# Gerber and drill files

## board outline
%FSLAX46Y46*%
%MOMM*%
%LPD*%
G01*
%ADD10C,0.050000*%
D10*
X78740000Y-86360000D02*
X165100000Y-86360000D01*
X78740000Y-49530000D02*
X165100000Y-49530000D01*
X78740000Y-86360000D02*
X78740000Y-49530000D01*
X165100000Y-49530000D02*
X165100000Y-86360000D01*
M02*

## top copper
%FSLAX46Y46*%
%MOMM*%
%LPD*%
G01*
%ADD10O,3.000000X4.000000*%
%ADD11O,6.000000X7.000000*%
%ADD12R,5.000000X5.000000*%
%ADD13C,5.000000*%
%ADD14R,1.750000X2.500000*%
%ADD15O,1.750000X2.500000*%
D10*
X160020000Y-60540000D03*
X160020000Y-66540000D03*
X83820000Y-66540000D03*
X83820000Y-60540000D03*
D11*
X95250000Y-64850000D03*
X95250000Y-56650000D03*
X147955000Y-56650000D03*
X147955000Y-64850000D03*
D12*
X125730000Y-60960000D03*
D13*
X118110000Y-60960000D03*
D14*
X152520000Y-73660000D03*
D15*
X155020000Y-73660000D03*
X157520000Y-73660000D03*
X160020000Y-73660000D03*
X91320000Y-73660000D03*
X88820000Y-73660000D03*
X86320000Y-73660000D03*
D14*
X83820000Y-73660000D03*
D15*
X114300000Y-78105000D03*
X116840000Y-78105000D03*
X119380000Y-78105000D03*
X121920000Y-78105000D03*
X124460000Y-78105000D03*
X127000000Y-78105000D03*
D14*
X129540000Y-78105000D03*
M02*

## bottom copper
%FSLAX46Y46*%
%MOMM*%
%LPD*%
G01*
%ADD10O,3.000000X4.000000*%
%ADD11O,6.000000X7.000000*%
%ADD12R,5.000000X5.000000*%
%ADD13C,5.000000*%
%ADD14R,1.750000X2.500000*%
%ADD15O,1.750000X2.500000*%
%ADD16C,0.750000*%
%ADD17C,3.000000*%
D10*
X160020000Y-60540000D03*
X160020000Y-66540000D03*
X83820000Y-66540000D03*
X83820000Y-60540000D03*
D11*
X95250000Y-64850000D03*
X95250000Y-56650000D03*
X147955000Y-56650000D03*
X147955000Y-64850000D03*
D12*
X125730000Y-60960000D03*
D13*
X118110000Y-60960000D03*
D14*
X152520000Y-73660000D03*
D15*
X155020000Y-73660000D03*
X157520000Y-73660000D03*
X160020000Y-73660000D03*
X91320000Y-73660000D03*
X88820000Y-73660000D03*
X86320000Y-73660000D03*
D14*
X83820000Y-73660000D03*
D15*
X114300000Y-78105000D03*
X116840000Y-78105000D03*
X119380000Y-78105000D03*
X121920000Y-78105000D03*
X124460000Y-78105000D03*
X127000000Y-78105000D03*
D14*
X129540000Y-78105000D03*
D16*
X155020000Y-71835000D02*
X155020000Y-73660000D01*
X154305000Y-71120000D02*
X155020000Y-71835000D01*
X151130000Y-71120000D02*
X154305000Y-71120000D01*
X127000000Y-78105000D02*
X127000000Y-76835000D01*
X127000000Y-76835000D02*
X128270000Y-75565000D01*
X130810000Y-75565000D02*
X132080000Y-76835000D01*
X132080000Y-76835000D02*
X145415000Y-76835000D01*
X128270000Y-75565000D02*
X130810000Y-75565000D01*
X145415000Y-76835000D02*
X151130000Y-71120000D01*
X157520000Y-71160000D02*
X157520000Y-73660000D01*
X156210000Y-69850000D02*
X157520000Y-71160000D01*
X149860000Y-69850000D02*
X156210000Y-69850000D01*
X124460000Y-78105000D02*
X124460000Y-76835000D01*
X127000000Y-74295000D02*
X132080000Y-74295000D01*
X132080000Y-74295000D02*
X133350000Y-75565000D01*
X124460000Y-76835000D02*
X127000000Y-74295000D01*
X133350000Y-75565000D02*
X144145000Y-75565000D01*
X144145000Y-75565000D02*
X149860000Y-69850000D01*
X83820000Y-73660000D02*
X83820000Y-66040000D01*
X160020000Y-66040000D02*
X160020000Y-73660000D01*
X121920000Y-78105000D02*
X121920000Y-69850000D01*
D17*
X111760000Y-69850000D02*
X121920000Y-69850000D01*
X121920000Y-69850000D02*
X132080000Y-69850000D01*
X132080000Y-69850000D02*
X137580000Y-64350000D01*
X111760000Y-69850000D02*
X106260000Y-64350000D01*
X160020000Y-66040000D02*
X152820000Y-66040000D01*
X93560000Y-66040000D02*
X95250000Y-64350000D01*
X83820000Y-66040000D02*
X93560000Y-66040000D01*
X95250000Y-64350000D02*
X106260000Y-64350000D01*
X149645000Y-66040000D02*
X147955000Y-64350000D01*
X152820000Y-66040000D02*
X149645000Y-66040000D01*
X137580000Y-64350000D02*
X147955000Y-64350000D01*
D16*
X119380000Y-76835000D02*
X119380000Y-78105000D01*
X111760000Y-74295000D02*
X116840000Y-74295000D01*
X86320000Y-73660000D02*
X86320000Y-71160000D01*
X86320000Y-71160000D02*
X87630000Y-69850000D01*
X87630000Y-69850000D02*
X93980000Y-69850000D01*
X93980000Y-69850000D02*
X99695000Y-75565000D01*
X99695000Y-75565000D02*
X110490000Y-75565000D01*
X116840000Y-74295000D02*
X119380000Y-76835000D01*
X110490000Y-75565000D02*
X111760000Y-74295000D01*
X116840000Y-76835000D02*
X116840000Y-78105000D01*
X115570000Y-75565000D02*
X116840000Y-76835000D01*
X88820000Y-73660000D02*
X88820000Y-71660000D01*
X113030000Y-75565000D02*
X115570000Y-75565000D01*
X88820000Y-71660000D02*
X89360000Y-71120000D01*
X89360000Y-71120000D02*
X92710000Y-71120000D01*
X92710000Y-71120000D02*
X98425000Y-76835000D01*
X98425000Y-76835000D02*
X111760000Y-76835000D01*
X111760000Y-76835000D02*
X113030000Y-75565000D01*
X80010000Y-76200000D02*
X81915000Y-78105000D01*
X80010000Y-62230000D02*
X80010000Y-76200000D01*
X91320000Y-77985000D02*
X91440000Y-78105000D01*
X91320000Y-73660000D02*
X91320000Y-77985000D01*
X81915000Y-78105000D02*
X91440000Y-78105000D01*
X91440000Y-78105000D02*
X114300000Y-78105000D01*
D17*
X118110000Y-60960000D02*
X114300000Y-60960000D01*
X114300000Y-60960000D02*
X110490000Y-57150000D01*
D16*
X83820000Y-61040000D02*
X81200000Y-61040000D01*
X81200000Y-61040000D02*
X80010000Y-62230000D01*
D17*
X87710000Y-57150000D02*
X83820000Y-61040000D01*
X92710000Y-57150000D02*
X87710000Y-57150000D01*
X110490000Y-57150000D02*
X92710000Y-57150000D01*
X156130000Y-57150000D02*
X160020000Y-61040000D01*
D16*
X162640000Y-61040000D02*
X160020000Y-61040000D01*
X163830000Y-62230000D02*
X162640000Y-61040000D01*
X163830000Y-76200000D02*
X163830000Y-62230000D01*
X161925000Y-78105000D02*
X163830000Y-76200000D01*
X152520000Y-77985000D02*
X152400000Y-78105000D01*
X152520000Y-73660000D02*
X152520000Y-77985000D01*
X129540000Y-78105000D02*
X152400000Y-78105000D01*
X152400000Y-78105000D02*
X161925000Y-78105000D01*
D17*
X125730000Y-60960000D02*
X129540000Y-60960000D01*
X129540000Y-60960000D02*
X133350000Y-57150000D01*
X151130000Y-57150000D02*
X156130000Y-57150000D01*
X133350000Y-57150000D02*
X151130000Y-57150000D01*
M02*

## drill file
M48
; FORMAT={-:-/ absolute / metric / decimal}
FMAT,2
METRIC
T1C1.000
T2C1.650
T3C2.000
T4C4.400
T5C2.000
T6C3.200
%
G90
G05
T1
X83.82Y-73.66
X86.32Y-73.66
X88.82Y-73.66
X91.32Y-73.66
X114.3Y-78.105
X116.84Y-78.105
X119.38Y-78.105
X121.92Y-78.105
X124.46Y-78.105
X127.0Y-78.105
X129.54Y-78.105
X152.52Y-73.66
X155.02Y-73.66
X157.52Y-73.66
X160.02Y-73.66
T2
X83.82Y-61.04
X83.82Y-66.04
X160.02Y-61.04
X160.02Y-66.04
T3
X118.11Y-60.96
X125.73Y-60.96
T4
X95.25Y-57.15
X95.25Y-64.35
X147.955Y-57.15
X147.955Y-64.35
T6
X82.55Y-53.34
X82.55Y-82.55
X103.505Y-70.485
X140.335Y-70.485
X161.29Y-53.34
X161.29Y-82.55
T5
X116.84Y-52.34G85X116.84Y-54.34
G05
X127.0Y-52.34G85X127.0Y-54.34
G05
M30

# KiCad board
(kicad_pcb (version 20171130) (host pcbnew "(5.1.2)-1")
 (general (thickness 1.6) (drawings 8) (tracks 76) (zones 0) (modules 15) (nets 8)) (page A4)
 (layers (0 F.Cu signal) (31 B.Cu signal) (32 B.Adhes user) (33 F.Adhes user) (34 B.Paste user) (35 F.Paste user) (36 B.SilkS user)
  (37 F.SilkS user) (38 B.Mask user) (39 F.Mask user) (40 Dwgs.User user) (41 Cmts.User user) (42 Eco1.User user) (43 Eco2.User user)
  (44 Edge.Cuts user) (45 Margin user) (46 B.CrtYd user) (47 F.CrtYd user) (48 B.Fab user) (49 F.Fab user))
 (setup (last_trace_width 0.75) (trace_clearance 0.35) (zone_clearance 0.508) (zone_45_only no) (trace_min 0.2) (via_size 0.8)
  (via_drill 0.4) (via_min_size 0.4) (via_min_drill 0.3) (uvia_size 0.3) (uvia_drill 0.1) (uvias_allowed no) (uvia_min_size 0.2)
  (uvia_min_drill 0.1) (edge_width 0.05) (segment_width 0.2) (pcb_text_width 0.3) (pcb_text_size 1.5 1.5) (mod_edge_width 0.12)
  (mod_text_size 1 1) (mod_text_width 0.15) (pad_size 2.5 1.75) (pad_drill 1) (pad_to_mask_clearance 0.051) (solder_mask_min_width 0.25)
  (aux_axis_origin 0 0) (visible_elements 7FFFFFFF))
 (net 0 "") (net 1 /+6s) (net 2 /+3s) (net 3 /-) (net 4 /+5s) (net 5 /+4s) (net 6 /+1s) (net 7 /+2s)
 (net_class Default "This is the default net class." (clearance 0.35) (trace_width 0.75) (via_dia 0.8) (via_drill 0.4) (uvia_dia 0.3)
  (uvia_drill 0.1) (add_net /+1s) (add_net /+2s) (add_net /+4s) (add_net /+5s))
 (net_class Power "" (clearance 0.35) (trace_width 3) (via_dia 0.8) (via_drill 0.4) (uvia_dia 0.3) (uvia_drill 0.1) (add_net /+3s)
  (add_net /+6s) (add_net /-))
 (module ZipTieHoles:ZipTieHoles (layer F.Cu) (at 121.92 53.34)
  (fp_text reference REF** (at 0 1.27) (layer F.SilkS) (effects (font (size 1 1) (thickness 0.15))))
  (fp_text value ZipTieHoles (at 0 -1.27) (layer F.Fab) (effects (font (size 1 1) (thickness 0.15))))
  (pad "" np_thru_hole oval (at 5.08 0) (size 2 4) (drill oval 2 4) (layers *.Cu *.Mask))
  (pad "" np_thru_hole oval (at -5.08 0) (size 2 4) (drill oval 2 4) (layers *.Cu *.Mask)))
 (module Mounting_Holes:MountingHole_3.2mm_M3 (layer F.Cu) (at 140.335 70.485)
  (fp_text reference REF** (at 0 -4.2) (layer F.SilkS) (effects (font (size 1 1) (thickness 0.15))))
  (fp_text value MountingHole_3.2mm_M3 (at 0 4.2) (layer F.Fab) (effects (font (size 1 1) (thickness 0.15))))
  (pad 1 np_thru_hole circle (at 0 0) (size 3.2 3.2) (drill 3.2) (layers *.Cu *.Mask)))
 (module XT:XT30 (layer F.Cu) (at 160.02 63.54 90)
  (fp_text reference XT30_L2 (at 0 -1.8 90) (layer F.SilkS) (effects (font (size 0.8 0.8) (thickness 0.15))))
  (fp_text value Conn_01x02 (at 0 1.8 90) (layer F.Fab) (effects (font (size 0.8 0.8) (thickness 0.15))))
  (pad 1 thru_hole oval (at 2.5 0 90) (size 4 3) (drill 1.65 (offset 0.5 0)) (layers *.Cu *.Mask) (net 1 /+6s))
  (pad 2 thru_hole oval (at -2.5 0 90) (size 4 3) (drill 1.65 (offset -0.5 0)) (layers *.Cu *.Mask) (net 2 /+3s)))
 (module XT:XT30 (layer F.Cu) (at 83.82 63.54 270)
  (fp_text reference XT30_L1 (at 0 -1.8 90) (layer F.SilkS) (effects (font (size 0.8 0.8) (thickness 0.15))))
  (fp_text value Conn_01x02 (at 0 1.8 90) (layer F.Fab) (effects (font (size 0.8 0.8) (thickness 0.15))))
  (pad 1 thru_hole oval (at 2.5 0 270) (size 4 3) (drill 1.65 (offset 0.5 0)) (layers *.Cu *.Mask) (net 2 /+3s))
  (pad 2 thru_hole oval (at -2.5 0 270) (size 4 3) (drill 1.65 (offset -0.5 0)) (layers *.Cu *.Mask) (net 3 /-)))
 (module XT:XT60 (layer F.Cu) (at 95.25 60.75 270)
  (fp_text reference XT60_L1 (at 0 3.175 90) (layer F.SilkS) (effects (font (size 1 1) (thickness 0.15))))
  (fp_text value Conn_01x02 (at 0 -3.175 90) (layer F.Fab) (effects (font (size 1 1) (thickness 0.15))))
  (pad 1 thru_hole oval (at 3.6 0 270) (size 7 6) (drill 4.4 (offset 0.5 0)) (layers *.Cu *.Mask) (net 2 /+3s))
  (pad 2 thru_hole oval (at -3.6 0 270) (size 7 6) (drill 4.4 (offset -0.5 0)) (layers *.Cu *.Mask) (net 3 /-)))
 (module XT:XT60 (layer F.Cu) (at 147.955 60.75 90)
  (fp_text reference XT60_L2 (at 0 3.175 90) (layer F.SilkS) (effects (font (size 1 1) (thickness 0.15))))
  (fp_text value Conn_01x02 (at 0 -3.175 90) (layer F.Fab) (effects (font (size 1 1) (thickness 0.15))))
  (pad 1 thru_hole oval (at 3.6 0 90) (size 7 6) (drill 4.4 (offset 0.5 0)) (layers *.Cu *.Mask) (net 1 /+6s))
  (pad 2 thru_hole oval (at -3.6 0 90) (size 7 6) (drill 4.4 (offset -0.5 0)) (layers *.Cu *.Mask) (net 2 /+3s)))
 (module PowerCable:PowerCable (layer F.Cu) (at 125.73 60.96 180)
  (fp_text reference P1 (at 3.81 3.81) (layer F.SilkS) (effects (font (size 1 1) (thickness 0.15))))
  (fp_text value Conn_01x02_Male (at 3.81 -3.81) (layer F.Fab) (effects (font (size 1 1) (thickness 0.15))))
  (pad 1 thru_hole rect (at 0 0 180) (size 5 5) (drill 2) (layers *.Cu *.Mask) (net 1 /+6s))
  (pad 2 thru_hole circle (at 7.62 0 180) (size 5 5) (drill 2) (layers *.Cu *.Mask) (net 3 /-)))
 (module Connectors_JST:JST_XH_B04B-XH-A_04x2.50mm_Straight (layer F.Cu) (at 152.52 73.66)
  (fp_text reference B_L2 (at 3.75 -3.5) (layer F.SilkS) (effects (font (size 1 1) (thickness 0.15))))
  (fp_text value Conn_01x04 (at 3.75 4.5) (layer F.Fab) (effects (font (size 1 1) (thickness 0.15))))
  (pad 1 thru_hole rect (at 0 0) (size 1.75 2.5) (drill 1) (layers *.Cu *.Mask) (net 1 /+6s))
  (pad 2 thru_hole oval (at 2.5 0) (size 1.75 2.5) (drill 1) (layers *.Cu *.Mask) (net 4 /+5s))
  (pad 3 thru_hole oval (at 5 0) (size 1.75 2.5) (drill 1) (layers *.Cu *.Mask) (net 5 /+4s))
  (pad 4 thru_hole oval (at 7.5 0) (size 1.75 2.5) (drill 1) (layers *.Cu *.Mask) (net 2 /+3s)))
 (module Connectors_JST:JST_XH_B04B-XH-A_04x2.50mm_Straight (layer F.Cu) (at 83.82 73.66)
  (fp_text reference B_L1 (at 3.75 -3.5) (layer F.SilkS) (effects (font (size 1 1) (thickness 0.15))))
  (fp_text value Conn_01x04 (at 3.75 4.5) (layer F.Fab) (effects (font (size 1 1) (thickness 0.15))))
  (pad 4 thru_hole oval (at 7.5 0) (size 1.75 2.5) (drill 1) (layers *.Cu *.Mask) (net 3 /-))
  (pad 3 thru_hole oval (at 5 0) (size 1.75 2.5) (drill 1) (layers *.Cu *.Mask) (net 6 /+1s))
  (pad 2 thru_hole oval (at 2.5 0) (size 1.75 2.5) (drill 1) (layers *.Cu *.Mask) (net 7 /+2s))
  (pad 1 thru_hole rect (at 0 0) (size 1.75 2.5) (drill 1) (layers *.Cu *.Mask) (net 2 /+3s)))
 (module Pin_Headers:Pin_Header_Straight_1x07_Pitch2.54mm (layer F.Cu) (at 129.54 78.105 270)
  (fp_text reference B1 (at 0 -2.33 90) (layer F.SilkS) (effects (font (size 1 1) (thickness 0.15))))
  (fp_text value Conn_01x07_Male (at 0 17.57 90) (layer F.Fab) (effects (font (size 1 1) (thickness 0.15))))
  (pad 7 thru_hole oval (at 0 15.24 270) (size 2.5 1.75) (drill 1) (layers *.Cu *.Mask) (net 3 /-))
  (pad 6 thru_hole oval (at 0 12.7 270) (size 2.5 1.75) (drill 1) (layers *.Cu *.Mask) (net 6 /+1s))
  (pad 5 thru_hole oval (at 0 10.16 270) (size 2.5 1.75) (drill 1) (layers *.Cu *.Mask) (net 7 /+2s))
  (pad 4 thru_hole oval (at 0 7.62 270) (size 2.5 1.75) (drill 1) (layers *.Cu *.Mask) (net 2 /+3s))
  (pad 3 thru_hole oval (at 0 5.08 270) (size 2.5 1.75) (drill 1) (layers *.Cu *.Mask) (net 5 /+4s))
  (pad 2 thru_hole oval (at 0 2.54 270) (size 2.5 1.75) (drill 1) (layers *.Cu *.Mask) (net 4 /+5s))
  (pad 1 thru_hole rect (at 0 0 270) (size 2.5 1.75) (drill 1) (layers *.Cu *.Mask) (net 1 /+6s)))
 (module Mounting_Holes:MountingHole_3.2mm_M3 (layer F.Cu) (at 161.29 53.34)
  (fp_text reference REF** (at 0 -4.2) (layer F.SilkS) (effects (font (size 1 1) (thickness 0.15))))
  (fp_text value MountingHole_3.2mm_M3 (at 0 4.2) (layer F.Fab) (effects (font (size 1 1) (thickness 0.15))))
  (pad 1 np_thru_hole circle (at 0 0) (size 3.2 3.2) (drill 3.2) (layers *.Cu *.Mask)))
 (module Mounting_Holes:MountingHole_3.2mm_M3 (layer F.Cu) (at 161.29 82.55)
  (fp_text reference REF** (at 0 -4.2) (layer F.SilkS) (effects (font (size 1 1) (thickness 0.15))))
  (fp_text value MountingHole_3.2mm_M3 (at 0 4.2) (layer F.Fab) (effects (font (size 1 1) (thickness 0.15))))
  (pad 1 np_thru_hole circle (at 0 0) (size 3.2 3.2) (drill 3.2) (layers *.Cu *.Mask)))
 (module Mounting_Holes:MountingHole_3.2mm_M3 (layer F.Cu) (at 82.55 82.55)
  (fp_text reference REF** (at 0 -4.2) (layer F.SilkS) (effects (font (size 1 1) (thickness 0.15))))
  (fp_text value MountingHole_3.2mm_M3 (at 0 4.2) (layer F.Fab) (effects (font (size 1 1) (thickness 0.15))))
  (pad 1 np_thru_hole circle (at 0 0) (size 3.2 3.2) (drill 3.2) (layers *.Cu *.Mask)))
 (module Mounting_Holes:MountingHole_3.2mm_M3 (layer F.Cu) (at 103.505 70.485)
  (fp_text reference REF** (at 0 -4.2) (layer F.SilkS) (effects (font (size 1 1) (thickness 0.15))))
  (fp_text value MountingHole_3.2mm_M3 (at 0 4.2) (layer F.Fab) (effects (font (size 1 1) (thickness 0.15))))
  (pad 1 np_thru_hole circle (at 0 0) (size 3.2 3.2) (drill 3.2) (layers *.Cu *.Mask)))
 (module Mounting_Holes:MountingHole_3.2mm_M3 (layer F.Cu) (at 82.55 53.34)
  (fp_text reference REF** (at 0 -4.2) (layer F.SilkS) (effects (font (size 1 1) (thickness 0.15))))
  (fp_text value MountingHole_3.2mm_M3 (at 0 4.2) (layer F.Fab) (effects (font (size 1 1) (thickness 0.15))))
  (pad 1 np_thru_hole circle (at 0 0) (size 3.2 3.2) (drill 3.2) (layers *.Cu *.Mask)))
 (gr_line (start 78.74 86.36) (end 165.1 86.36) (layer Edge.Cuts) (width 0.05))
 (gr_line (start 78.74 49.53) (end 165.1 49.53) (layer Edge.Cuts) (width 0.05))
 (gr_line (start 78.74 86.36) (end 78.74 49.53) (layer Edge.Cuts) (width 0.05))
 (gr_line (start 165.1 49.53) (end 165.1 86.36) (layer Edge.Cuts) (width 0.05))
 (segment (start 155.02 71.835) (end 155.02 73.66) (width 0.75) (layer B.Cu) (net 4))
 (segment (start 154.305 71.12) (end 155.02 71.835) (width 0.75) (layer B.Cu) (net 4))
 (segment (start 151.13 71.12) (end 154.305 71.12) (width 0.75) (layer B.Cu) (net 4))
 (segment (start 127 78.105) (end 127 76.835) (width 0.75) (layer B.Cu) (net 4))
 (segment (start 127 76.835) (end 128.27 75.565) (width 0.75) (layer B.Cu) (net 4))
 (segment (start 130.81 75.565) (end 132.08 76.835) (width 0.75) (layer B.Cu) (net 4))
 (segment (start 132.08 76.835) (end 145.415 76.835) (width 0.75) (layer B.Cu) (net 4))
 (segment (start 128.27 75.565) (end 130.81 75.565) (width 0.75) (layer B.Cu) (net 4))
 (segment (start 145.415 76.835) (end 151.13 71.12) (width 0.75) (layer B.Cu) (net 4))
 (segment (start 157.52 71.16) (end 157.52 73.66) (width 0.75) (layer B.Cu) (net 5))
 (segment (start 156.21 69.85) (end 157.52 71.16) (width 0.75) (layer B.Cu) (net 5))
 (segment (start 149.86 69.85) (end 156.21 69.85) (width 0.75) (layer B.Cu) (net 5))
 (segment (start 124.46 78.105) (end 124.46 76.835) (width 0.75) (layer B.Cu) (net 5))
 (segment (start 127 74.295) (end 132.08 74.295) (width 0.75) (layer B.Cu) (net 5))
 (segment (start 132.08 74.295) (end 133.35 75.565) (width 0.75) (layer B.Cu) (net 5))
 (segment (start 124.46 76.835) (end 127 74.295) (width 0.75) (layer B.Cu) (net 5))
 (segment (start 133.35 75.565) (end 144.145 75.565) (width 0.75) (layer B.Cu) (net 5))
 (segment (start 144.145 75.565) (end 149.86 69.85) (width 0.75) (layer B.Cu) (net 5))
 (segment (start 83.82 73.66) (end 83.82 66.04) (width 0.75) (layer B.Cu) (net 2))
 (segment (start 160.02 66.04) (end 160.02 73.66) (width 0.75) (layer B.Cu) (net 2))
 (segment (start 121.92 78.105) (end 121.92 69.85) (width 0.75) (layer B.Cu) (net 2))
 (segment (start 111.76 69.85) (end 121.92 69.85) (width 3) (layer B.Cu) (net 2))
 (segment (start 121.92 69.85) (end 132.08 69.85) (width 3) (layer B.Cu) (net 2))
 (segment (start 132.08 69.85) (end 137.58 64.35) (width 3) (layer B.Cu) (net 2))
 (segment (start 111.76 69.85) (end 106.26 64.35) (width 3) (layer B.Cu) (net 2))
 (segment (start 160.02 66.04) (end 152.82 66.04) (width 3) (layer B.Cu) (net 2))
 (segment (start 93.56 66.04) (end 95.25 64.35) (width 3) (layer B.Cu) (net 2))
 (segment (start 83.82 66.04) (end 93.56 66.04) (width 3) (layer B.Cu) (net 2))
 (segment (start 95.25 64.35) (end 106.26 64.35) (width 3) (layer B.Cu) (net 2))
 (segment (start 149.645 66.04) (end 147.955 64.35) (width 3) (layer B.Cu) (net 2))
 (segment (start 152.82 66.04) (end 149.645 66.04) (width 3) (layer B.Cu) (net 2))
 (segment (start 137.58 64.35) (end 147.955 64.35) (width 3) (layer B.Cu) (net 2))
 (segment (start 119.38 76.835) (end 119.38 78.105) (width 0.75) (layer B.Cu) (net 7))
 (segment (start 111.76 74.295) (end 116.84 74.295) (width 0.75) (layer B.Cu) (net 7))
 (segment (start 86.32 73.66) (end 86.32 71.16) (width 0.75) (layer B.Cu) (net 7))
 (segment (start 86.32 71.16) (end 87.63 69.85) (width 0.75) (layer B.Cu) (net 7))
 (segment (start 87.63 69.85) (end 93.98 69.85) (width 0.75) (layer B.Cu) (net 7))
 (segment (start 93.98 69.85) (end 99.695 75.565) (width 0.75) (layer B.Cu) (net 7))
 (segment (start 99.695 75.565) (end 110.49 75.565) (width 0.75) (layer B.Cu) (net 7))
 (segment (start 116.84 74.295) (end 119.38 76.835) (width 0.75) (layer B.Cu) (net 7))
 (segment (start 110.49 75.565) (end 111.76 74.295) (width 0.75) (layer B.Cu) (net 7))
 (segment (start 116.84 76.835) (end 116.84 78.105) (width 0.75) (layer B.Cu) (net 6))
 (segment (start 115.57 75.565) (end 116.84 76.835) (width 0.75) (layer B.Cu) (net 6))
 (segment (start 88.82 73.66) (end 88.82 71.66) (width 0.75) (layer B.Cu) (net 6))
 (segment (start 113.03 75.565) (end 115.57 75.565) (width 0.75) (layer B.Cu) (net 6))
 (segment (start 88.82 71.66) (end 89.36 71.12) (width 0.75) (layer B.Cu) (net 6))
 (segment (start 89.36 71.12) (end 92.71 71.12) (width 0.75) (layer B.Cu) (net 6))
 (segment (start 92.71 71.12) (end 98.425 76.835) (width 0.75) (layer B.Cu) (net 6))
 (segment (start 98.425 76.835) (end 111.76 76.835) (width 0.75) (layer B.Cu) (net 6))
 (segment (start 111.76 76.835) (end 113.03 75.565) (width 0.75) (layer B.Cu) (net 6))
 (segment (start 80.01 76.2) (end 81.915 78.105) (width 0.75) (layer B.Cu) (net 3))
 (segment (start 80.01 62.23) (end 80.01 76.2) (width 0.75) (layer B.Cu) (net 3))
 (segment (start 91.32 77.985) (end 91.44 78.105) (width 0.75) (layer B.Cu) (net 3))
 (segment (start 91.32 73.66) (end 91.32 77.985) (width 0.75) (layer B.Cu) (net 3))
 (segment (start 81.915 78.105) (end 91.44 78.105) (width 0.75) (layer B.Cu) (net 3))
 (segment (start 91.44 78.105) (end 114.3 78.105) (width 0.75) (layer B.Cu) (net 3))
 (segment (start 118.11 60.96) (end 114.3 60.96) (width 3) (layer B.Cu) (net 3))
 (segment (start 114.3 60.96) (end 110.49 57.15) (width 3) (layer B.Cu) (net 3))
 (segment (start 83.82 61.04) (end 81.2 61.04) (width 0.75) (layer B.Cu) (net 3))
 (segment (start 81.2 61.04) (end 80.01 62.23) (width 0.75) (layer B.Cu) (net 3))
 (segment (start 87.71 57.15) (end 83.82 61.04) (width 3) (layer B.Cu) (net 3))
 (segment (start 92.71 57.15) (end 87.71 57.15) (width 3) (layer B.Cu) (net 3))
 (segment (start 110.49 57.15) (end 92.71 57.15) (width 3) (layer B.Cu) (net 3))
 (segment (start 156.13 57.15) (end 160.02 61.04) (width 3) (layer B.Cu) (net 1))
 (segment (start 162.64 61.04) (end 160.02 61.04) (width 0.75) (layer B.Cu) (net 1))
 (segment (start 163.83 62.23) (end 162.64 61.04) (width 0.75) (layer B.Cu) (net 1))
 (segment (start 163.83 76.2) (end 163.83 62.23) (width 0.75) (layer B.Cu) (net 1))
 (segment (start 161.925 78.105) (end 163.83 76.2) (width 0.75) (layer B.Cu) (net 1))
 (segment (start 152.52 77.985) (end 152.4 78.105) (width 0.75) (layer B.Cu) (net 1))
 (segment (start 152.52 73.66) (end 152.52 77.985) (width 0.75) (layer B.Cu) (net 1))
 (segment (start 129.54 78.105) (end 152.4 78.105) (width 0.75) (layer B.Cu) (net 1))
 (segment (start 152.4 78.105) (end 161.925 78.105) (width 0.75) (layer B.Cu) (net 1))
 (segment (start 125.73 60.96) (end 129.54 60.96) (width 3) (layer B.Cu) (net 1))
 (segment (start 129.54 60.96) (end 133.35 57.15) (width 3) (layer B.Cu) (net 1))
 (segment (start 151.13 57.15) (end 156.13 57.15) (width 3) (layer B.Cu) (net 1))
 (segment (start 133.35 57.15) (end 151.13 57.15) (width 3) (layer B.Cu) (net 1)))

